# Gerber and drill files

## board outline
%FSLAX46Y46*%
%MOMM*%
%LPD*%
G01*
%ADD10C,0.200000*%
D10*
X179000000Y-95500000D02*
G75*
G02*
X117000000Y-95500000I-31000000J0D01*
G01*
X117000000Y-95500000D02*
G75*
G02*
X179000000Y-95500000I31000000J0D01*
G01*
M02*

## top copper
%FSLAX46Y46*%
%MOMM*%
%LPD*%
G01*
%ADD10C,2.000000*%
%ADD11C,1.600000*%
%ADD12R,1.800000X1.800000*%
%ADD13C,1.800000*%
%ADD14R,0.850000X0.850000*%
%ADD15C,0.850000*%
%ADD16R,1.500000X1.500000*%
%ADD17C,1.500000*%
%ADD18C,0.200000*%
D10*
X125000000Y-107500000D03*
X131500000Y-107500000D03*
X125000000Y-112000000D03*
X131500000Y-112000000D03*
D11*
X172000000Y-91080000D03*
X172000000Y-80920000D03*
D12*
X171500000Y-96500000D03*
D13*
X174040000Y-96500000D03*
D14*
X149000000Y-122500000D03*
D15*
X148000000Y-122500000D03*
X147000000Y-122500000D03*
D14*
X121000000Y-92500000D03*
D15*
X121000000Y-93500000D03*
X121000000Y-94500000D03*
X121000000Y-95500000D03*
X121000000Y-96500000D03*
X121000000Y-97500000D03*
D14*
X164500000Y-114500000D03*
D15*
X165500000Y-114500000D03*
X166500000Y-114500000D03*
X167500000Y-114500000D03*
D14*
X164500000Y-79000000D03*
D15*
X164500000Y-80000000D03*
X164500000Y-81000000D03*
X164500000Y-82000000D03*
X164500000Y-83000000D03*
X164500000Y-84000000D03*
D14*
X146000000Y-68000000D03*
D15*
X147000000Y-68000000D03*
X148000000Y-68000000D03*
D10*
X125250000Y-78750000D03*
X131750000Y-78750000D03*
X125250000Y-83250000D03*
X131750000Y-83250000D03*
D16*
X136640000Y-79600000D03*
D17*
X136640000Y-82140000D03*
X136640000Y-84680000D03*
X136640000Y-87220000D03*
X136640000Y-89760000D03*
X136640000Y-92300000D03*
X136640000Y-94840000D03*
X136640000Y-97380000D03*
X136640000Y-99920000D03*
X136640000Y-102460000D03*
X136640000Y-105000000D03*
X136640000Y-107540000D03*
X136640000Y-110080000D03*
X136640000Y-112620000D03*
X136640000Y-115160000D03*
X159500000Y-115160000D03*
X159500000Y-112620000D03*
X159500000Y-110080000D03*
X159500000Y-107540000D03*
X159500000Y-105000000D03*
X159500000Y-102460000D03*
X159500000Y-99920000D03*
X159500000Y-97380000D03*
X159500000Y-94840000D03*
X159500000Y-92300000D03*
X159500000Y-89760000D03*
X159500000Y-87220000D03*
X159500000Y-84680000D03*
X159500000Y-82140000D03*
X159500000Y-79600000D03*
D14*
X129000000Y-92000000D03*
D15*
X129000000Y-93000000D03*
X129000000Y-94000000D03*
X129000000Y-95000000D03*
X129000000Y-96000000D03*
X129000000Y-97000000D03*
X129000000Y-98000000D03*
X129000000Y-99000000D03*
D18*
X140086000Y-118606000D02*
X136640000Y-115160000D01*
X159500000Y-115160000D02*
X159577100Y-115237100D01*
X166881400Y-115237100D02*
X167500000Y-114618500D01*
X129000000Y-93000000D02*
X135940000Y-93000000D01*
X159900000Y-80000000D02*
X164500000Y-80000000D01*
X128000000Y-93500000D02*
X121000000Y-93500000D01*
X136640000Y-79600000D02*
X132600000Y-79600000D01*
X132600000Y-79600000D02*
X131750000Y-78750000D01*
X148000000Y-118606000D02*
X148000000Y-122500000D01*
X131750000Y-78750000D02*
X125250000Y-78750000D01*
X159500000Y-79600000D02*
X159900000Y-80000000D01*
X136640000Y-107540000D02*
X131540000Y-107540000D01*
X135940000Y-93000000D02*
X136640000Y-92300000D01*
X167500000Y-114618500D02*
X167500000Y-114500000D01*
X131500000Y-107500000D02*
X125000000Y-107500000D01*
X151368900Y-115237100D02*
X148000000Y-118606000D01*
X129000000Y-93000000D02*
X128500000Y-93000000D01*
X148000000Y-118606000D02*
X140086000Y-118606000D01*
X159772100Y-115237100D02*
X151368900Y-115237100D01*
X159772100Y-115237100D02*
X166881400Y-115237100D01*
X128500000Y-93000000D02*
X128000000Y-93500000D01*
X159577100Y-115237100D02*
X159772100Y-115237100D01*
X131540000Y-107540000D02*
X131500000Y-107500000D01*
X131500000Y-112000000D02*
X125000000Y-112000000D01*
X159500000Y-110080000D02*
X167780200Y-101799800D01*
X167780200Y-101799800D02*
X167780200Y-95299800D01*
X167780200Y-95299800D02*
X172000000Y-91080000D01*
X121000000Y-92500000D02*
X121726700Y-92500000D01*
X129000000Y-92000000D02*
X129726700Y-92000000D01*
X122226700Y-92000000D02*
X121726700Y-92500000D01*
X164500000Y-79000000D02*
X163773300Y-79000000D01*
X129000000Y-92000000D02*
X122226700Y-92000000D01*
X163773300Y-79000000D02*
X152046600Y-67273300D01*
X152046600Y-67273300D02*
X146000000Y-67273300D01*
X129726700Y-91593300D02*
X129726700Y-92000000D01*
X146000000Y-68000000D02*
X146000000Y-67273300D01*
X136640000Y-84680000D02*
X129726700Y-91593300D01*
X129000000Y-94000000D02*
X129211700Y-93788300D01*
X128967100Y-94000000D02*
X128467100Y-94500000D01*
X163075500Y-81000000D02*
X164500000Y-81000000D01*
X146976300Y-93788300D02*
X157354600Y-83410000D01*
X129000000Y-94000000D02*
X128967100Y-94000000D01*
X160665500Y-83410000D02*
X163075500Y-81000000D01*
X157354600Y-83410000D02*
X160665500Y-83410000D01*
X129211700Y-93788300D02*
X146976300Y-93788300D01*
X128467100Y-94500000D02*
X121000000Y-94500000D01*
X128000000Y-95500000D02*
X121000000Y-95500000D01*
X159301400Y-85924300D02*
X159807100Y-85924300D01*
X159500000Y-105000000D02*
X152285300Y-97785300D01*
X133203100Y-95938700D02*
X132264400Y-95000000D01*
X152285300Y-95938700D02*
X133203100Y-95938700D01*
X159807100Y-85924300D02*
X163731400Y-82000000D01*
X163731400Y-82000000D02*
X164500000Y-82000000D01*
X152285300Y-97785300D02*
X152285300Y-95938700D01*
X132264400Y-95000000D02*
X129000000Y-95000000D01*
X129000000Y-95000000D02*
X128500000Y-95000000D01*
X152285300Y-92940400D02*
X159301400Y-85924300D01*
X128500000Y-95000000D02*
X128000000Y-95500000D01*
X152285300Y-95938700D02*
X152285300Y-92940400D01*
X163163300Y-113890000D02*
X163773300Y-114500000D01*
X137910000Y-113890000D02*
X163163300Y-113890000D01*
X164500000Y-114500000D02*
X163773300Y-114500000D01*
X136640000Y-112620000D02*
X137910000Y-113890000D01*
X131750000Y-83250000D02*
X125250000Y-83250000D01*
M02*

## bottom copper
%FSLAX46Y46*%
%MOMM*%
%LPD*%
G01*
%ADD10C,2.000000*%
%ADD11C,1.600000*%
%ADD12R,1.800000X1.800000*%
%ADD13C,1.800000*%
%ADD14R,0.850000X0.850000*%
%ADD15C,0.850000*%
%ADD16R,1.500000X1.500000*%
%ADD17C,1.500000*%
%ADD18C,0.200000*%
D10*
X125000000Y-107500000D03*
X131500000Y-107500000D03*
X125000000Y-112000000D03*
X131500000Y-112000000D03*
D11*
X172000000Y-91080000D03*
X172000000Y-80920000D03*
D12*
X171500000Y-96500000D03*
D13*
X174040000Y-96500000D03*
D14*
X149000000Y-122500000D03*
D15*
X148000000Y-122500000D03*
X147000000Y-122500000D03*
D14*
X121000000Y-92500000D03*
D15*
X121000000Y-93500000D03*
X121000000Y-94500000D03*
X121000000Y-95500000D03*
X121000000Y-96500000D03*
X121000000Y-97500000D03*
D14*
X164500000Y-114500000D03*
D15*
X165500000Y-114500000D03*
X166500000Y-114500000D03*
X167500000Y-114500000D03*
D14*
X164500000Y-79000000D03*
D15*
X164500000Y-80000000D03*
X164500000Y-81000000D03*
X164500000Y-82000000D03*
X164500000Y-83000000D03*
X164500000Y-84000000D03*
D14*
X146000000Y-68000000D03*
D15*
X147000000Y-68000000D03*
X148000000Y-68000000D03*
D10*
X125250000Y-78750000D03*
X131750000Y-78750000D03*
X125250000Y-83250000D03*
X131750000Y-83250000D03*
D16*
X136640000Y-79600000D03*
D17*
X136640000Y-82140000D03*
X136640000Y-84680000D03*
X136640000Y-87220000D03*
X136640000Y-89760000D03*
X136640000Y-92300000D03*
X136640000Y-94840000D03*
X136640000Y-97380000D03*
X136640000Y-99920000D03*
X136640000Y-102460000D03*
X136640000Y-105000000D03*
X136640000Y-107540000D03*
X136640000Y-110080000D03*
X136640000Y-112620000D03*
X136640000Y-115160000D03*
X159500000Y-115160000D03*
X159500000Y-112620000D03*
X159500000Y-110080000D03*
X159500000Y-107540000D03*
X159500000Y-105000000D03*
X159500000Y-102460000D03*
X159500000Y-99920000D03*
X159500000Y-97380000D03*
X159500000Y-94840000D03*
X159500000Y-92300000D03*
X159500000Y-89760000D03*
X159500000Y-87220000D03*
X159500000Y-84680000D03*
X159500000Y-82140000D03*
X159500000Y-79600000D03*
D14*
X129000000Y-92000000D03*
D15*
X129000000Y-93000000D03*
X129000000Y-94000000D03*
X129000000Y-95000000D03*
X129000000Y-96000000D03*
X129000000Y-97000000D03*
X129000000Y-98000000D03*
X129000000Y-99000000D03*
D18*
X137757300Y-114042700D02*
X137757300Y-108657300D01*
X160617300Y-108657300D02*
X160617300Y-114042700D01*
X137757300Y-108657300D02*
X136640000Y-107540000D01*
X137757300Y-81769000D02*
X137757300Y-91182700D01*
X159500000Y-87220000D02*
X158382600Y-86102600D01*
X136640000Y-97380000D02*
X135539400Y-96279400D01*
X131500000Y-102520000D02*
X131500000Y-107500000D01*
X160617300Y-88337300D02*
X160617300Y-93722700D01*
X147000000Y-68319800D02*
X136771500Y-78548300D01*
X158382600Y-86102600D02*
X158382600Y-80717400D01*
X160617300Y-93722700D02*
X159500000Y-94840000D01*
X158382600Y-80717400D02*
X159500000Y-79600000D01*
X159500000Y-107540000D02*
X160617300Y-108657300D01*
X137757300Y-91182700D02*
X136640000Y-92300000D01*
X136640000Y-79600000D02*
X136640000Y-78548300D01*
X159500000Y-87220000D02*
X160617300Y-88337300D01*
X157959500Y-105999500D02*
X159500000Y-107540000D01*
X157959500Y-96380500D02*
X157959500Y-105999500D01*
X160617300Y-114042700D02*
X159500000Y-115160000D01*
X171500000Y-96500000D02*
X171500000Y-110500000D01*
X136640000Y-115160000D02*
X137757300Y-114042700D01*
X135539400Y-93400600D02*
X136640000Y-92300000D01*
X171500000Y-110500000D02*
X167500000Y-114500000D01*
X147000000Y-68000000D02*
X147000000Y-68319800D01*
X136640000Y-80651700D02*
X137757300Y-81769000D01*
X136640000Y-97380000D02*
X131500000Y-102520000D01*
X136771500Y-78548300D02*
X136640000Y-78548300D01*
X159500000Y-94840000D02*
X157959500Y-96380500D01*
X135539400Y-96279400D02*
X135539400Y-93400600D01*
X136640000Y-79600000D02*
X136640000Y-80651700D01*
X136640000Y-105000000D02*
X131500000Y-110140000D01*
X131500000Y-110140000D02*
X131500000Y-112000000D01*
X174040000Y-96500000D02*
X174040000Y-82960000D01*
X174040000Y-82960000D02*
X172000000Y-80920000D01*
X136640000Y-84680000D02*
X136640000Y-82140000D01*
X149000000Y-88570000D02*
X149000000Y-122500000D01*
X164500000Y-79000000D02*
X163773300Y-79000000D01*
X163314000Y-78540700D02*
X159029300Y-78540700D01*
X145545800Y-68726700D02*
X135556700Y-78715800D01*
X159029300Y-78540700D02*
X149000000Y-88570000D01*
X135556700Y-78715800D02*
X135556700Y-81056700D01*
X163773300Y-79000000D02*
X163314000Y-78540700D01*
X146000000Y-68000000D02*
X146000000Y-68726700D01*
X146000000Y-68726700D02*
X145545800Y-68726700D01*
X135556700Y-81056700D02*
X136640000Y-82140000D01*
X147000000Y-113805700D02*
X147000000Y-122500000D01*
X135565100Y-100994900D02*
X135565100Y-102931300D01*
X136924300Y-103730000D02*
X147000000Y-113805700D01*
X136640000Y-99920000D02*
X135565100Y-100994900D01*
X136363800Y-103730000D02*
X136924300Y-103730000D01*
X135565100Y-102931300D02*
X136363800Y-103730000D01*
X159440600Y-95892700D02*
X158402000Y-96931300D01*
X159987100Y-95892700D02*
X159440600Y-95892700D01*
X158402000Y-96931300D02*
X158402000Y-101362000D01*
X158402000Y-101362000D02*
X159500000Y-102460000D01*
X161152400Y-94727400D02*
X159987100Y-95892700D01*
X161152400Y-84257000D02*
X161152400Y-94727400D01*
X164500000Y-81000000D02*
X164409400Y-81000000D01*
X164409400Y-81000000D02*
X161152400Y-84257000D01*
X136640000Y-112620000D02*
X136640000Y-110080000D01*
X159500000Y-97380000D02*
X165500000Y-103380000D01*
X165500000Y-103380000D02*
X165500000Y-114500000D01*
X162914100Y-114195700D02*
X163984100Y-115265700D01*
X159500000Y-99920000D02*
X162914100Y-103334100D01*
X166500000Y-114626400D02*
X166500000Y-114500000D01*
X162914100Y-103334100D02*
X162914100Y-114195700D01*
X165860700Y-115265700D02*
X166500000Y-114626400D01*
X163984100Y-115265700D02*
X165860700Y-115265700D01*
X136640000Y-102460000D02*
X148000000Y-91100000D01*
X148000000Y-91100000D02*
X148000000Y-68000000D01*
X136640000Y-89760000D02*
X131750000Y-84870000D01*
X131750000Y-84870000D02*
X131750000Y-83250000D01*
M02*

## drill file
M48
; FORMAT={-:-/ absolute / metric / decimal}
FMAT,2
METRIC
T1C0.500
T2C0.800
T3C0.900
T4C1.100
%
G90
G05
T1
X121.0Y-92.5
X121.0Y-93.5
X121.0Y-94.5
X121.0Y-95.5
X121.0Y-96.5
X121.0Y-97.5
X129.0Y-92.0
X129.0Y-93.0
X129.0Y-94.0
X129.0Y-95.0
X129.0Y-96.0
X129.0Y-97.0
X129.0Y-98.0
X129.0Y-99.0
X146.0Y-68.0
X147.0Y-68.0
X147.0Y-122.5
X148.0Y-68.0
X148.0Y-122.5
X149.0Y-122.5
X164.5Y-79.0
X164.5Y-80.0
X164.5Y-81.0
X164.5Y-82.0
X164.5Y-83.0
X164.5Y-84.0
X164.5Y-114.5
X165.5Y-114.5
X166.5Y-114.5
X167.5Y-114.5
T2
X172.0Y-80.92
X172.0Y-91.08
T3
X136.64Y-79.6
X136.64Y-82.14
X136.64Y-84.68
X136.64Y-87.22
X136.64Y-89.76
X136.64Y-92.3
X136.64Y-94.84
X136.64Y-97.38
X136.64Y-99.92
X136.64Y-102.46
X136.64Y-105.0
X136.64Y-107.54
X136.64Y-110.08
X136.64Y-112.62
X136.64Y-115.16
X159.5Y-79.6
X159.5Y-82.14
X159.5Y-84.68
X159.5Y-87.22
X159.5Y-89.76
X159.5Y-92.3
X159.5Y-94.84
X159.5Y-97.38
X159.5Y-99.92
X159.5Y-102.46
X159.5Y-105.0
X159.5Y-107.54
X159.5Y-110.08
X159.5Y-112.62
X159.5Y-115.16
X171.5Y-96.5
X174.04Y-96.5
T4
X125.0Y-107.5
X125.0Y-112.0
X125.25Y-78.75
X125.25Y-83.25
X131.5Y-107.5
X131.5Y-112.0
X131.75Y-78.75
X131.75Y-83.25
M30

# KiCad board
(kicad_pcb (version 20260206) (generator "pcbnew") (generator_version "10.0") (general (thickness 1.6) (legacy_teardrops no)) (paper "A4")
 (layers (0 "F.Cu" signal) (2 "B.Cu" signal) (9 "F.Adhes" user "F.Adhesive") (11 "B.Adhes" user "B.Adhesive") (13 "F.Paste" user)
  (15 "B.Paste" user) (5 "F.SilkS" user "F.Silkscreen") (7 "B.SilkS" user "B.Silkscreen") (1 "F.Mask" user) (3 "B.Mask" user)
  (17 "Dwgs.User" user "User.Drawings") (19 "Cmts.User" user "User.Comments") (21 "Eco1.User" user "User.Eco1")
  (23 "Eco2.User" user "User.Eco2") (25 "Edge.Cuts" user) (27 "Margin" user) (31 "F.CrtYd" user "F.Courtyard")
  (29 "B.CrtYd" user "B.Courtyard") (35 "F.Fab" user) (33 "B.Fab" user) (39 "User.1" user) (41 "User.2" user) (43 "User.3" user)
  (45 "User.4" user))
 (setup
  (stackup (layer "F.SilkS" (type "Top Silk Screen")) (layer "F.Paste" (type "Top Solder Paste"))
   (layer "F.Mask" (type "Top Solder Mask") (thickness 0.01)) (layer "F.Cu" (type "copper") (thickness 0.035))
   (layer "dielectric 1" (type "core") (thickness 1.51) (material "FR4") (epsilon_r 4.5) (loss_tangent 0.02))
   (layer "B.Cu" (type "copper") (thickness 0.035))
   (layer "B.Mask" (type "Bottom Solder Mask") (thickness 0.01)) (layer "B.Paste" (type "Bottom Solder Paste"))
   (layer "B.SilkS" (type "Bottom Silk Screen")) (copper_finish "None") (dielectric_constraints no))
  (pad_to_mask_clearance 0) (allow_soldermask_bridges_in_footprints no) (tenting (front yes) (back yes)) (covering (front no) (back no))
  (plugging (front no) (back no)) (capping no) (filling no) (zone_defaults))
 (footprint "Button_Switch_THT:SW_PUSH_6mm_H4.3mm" (layer "F.Cu") (at 125 107.5)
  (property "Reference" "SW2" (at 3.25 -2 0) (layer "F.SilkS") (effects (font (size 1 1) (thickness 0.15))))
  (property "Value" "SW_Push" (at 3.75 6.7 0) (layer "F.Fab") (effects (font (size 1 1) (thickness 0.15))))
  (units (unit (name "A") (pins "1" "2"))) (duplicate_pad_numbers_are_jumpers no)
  (pad "1" thru_hole circle (at 0 0 90) (size 2 2) (drill 1.1) (layers "*.Cu" "*.Mask") (remove_unused_layers no) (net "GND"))
  (pad "1" thru_hole circle (at 6.5 0 90) (size 2 2) (drill 1.1) (layers "*.Cu" "*.Mask") (remove_unused_layers no) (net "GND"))
  (pad "2" thru_hole circle (at 0 4.5 90) (size 2 2) (drill 1.1) (layers "*.Cu" "*.Mask") (remove_unused_layers no) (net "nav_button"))
  (pad "2" thru_hole circle (at 6.5 4.5 90) (size 2 2) (drill 1.1) (layers "*.Cu" "*.Mask") (remove_unused_layers no) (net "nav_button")))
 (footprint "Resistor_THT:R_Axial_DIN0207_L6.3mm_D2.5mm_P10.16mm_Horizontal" (layer "F.Cu") (at 172 91.08 90)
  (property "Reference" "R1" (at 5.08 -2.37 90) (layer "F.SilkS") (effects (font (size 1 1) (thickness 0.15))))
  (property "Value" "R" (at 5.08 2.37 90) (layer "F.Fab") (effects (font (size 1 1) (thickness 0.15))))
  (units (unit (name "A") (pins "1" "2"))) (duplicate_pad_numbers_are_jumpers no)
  (pad "1" thru_hole circle (at 0 0 90) (size 1.6 1.6) (drill 0.8) (layers "*.Cu" "*.Mask") (remove_unused_layers no) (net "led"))
  (pad "2" thru_hole circle (at 10.16 0 90) (size 1.6 1.6) (drill 0.8) (layers "*.Cu" "*.Mask") (remove_unused_layers no) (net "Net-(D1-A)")))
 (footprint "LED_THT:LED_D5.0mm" (layer "F.Cu") (at 171.5 96.5)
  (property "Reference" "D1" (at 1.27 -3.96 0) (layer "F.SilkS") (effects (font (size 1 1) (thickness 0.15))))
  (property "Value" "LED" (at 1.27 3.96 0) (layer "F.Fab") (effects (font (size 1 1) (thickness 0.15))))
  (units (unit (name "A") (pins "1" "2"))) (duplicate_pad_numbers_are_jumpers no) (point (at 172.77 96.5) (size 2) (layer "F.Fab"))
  (pad "1" thru_hole rect (at 0 0) (size 1.8 1.8) (drill 0.9) (layers "*.Cu" "*.Mask") (remove_unused_layers no) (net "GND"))
  (pad "2" thru_hole circle (at 2.54 0) (size 1.8 1.8) (drill 0.9) (layers "*.Cu" "*.Mask") (remove_unused_layers no) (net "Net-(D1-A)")))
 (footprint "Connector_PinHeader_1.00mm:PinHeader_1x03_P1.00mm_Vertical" (layer "F.Cu") (at 149 122.5 -90)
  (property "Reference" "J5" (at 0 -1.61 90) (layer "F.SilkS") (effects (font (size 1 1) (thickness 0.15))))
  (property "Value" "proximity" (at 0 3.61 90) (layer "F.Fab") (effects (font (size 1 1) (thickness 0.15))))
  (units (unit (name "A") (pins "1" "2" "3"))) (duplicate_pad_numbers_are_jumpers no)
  (pad "1" thru_hole rect (at 0 0 270) (size 0.85 0.85) (drill 0.5) (layers "*.Cu" "*.Mask") (remove_unused_layers no) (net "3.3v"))
  (pad "2" thru_hole circle (at 0 1 270) (size 0.85 0.85) (drill 0.5) (layers "*.Cu" "*.Mask") (remove_unused_layers no) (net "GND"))
  (pad "3" thru_hole circle (at 0 2 270) (size 0.85 0.85) (drill 0.5) (layers "*.Cu" "*.Mask") (remove_unused_layers no) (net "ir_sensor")))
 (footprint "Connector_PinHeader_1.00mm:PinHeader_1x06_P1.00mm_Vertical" (layer "F.Cu") (at 121 92.5)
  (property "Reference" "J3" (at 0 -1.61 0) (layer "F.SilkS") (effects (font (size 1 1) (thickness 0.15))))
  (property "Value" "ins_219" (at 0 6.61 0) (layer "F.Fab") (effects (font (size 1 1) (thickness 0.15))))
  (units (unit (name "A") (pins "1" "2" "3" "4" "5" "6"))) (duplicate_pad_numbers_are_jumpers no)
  (pad "1" thru_hole rect (at 0 0) (size 0.85 0.85) (drill 0.5) (layers "*.Cu" "*.Mask") (remove_unused_layers no) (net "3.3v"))
  (pad "2" thru_hole circle (at 0 1) (size 0.85 0.85) (drill 0.5) (layers "*.Cu" "*.Mask") (remove_unused_layers no) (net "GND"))
  (pad "3" thru_hole circle (at 0 2) (size 0.85 0.85) (drill 0.5) (layers "*.Cu" "*.Mask") (remove_unused_layers no) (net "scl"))
  (pad "4" thru_hole circle (at 0 3) (size 0.85 0.85) (drill 0.5) (layers "*.Cu" "*.Mask") (remove_unused_layers no) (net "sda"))
  (pad "5" thru_hole circle (at 0 4) (size 0.85 0.85) (drill 0.5) (layers "*.Cu" "*.Mask") (remove_unused_layers no)
   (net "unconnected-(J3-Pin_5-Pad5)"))
  (pad "6" thru_hole circle (at 0 5) (size 0.85 0.85) (drill 0.5) (layers "*.Cu" "*.Mask") (remove_unused_layers no)
   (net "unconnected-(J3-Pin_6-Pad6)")))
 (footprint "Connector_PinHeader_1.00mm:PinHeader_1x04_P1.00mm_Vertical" (layer "F.Cu") (at 164.5 114.5 90)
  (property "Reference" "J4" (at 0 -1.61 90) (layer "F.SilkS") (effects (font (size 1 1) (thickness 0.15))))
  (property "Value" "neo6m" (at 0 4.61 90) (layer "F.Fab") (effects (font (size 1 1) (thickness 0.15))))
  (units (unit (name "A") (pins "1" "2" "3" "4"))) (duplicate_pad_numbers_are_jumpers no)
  (pad "1" thru_hole rect (at 0 0 90) (size 0.85 0.85) (drill 0.5) (layers "*.Cu" "*.Mask") (remove_unused_layers no) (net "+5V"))
  (pad "2" thru_hole circle (at 0 1 90) (size 0.85 0.85) (drill 0.5) (layers "*.Cu" "*.Mask") (remove_unused_layers no) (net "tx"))
  (pad "3" thru_hole circle (at 0 2 90) (size 0.85 0.85) (drill 0.5) (layers "*.Cu" "*.Mask") (remove_unused_layers no) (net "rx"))
  (pad "4" thru_hole circle (at 0 3 90) (size 0.85 0.85) (drill 0.5) (layers "*.Cu" "*.Mask") (remove_unused_layers no) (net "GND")))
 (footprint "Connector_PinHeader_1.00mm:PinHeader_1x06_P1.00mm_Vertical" (layer "F.Cu") (at 164.5 79)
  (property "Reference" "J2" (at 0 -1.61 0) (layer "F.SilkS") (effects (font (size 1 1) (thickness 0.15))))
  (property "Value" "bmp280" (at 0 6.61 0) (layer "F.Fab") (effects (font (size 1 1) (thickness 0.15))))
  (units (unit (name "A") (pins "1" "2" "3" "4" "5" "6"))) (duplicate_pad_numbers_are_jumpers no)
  (pad "1" thru_hole rect (at 0 0) (size 0.85 0.85) (drill 0.5) (layers "*.Cu" "*.Mask") (remove_unused_layers no) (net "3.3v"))
  (pad "2" thru_hole circle (at 0 1) (size 0.85 0.85) (drill 0.5) (layers "*.Cu" "*.Mask") (remove_unused_layers no) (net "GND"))
  (pad "3" thru_hole circle (at 0 2) (size 0.85 0.85) (drill 0.5) (layers "*.Cu" "*.Mask") (remove_unused_layers no) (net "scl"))
  (pad "4" thru_hole circle (at 0 3) (size 0.85 0.85) (drill 0.5) (layers "*.Cu" "*.Mask") (remove_unused_layers no) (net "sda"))
  (pad "5" thru_hole circle (at 0 4) (size 0.85 0.85) (drill 0.5) (layers "*.Cu" "*.Mask") (remove_unused_layers no)
   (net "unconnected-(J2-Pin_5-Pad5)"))
  (pad "6" thru_hole circle (at 0 5) (size 0.85 0.85) (drill 0.5) (layers "*.Cu" "*.Mask") (remove_unused_layers no)
   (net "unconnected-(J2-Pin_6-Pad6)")))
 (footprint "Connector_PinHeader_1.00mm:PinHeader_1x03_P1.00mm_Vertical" (layer "F.Cu") (at 146 68 90)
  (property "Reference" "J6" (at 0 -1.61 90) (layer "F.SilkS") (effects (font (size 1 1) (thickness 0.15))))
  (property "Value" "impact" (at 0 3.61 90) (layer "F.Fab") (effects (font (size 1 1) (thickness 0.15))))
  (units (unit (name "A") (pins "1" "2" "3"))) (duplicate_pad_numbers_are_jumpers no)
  (pad "1" thru_hole rect (at 0 0 90) (size 0.85 0.85) (drill 0.5) (layers "*.Cu" "*.Mask") (remove_unused_layers no) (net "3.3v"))
  (pad "2" thru_hole circle (at 0 1 90) (size 0.85 0.85) (drill 0.5) (layers "*.Cu" "*.Mask") (remove_unused_layers no) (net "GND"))
  (pad "3" thru_hole circle (at 0 2 90) (size 0.85 0.85) (drill 0.5) (layers "*.Cu" "*.Mask") (remove_unused_layers no) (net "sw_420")))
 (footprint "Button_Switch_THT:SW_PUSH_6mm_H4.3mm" (layer "F.Cu") (at 125.25 78.75)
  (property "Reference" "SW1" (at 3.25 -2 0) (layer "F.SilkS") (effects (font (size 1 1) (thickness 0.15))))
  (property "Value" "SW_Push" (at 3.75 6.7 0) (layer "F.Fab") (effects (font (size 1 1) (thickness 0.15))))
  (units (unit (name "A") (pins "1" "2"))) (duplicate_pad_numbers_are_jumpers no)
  (pad "1" thru_hole circle (at 0 0 90) (size 2 2) (drill 1.1) (layers "*.Cu" "*.Mask") (remove_unused_layers no) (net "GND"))
  (pad "1" thru_hole circle (at 6.5 0 90) (size 2 2) (drill 1.1) (layers "*.Cu" "*.Mask") (remove_unused_layers no) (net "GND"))
  (pad "2" thru_hole circle (at 0 4.5 90) (size 2 2) (drill 1.1) (layers "*.Cu" "*.Mask") (remove_unused_layers no) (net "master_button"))
  (pad "2" thru_hole circle (at 6.5 4.5 90) (size 2 2) (drill 1.1) (layers "*.Cu" "*.Mask") (remove_unused_layers no) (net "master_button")))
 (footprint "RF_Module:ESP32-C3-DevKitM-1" (layer "F.Cu") (at 136.64 79.6)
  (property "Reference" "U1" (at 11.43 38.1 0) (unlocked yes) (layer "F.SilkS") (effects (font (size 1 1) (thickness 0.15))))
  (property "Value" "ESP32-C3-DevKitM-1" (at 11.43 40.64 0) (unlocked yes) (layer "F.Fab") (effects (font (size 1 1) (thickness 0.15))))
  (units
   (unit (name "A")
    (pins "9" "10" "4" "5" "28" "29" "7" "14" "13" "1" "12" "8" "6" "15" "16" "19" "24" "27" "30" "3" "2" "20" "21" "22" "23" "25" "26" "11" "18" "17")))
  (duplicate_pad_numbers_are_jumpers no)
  (pad "1" thru_hole rect (at 0 0) (size 1.5 1.5) (drill 0.9) (layers "*.Cu" "*.Mask") (remove_unused_layers yes) (keep_end_layers yes)
   (zone_layer_connections) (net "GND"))
  (pad "2" thru_hole circle (at 0 2.54) (size 1.5 1.5) (drill 0.9) (layers "*.Cu" "*.Mask") (remove_unused_layers yes) (keep_end_layers yes)
   (zone_layer_connections) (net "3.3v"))
  (pad "3" thru_hole circle (at 0 5.08) (size 1.5 1.5) (drill 0.9) (layers "*.Cu" "*.Mask") (remove_unused_layers yes) (keep_end_layers yes)
   (zone_layer_connections) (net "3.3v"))
  (pad "4" thru_hole circle (at 0 7.62) (size 1.5 1.5) (drill 0.9) (layers "*.Cu" "*.Mask") (remove_unused_layers yes) (keep_end_layers yes)
   (zone_layer_connections) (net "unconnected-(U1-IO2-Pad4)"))
  (pad "5" thru_hole circle (at 0 10.16) (size 1.5 1.5) (drill 0.9) (layers "*.Cu" "*.Mask") (remove_unused_layers yes)
   (keep_end_layers yes) (zone_layer_connections) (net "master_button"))
  (pad "6" thru_hole circle (at 0 12.7) (size 1.5 1.5) (drill 0.9) (layers "*.Cu" "*.Mask") (remove_unused_layers yes) (keep_end_layers yes)
   (zone_layer_connections) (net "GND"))
  (pad "7" thru_hole circle (at 0 15.24) (size 1.5 1.5) (drill 0.9) (layers "*.Cu" "*.Mask") (remove_unused_layers yes)
   (keep_end_layers yes) (zone_layer_connections) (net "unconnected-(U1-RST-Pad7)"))
  (pad "8" thru_hole circle (at 0 17.78) (size 1.5 1.5) (drill 0.9) (layers "*.Cu" "*.Mask") (remove_unused_layers yes)
   (keep_end_layers yes) (zone_layer_connections) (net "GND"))
  (pad "9" thru_hole circle (at 0 20.32) (size 1.5 1.5) (drill 0.9) (layers "*.Cu" "*.Mask") (remove_unused_layers yes)
   (keep_end_layers yes) (zone_layer_connections) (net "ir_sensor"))
  (pad "10" thru_hole circle (at 0 22.86) (size 1.5 1.5) (drill 0.9) (layers "*.Cu" "*.Mask") (remove_unused_layers yes)
   (keep_end_layers yes) (zone_layer_connections) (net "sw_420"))
  (pad "11" thru_hole circle (at 0 25.4) (size 1.5 1.5) (drill 0.9) (layers "*.Cu" "*.Mask") (remove_unused_layers yes)
   (keep_end_layers yes) (zone_layer_connections) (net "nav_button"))
  (pad "12" thru_hole circle (at 0 27.94) (size 1.5 1.5) (drill 0.9) (layers "*.Cu" "*.Mask") (remove_unused_layers yes)
   (keep_end_layers yes) (zone_layer_connections) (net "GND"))
  (pad "13" thru_hole circle (at 0 30.48) (size 1.5 1.5) (drill 0.9) (layers "*.Cu" "*.Mask") (remove_unused_layers yes)
   (keep_end_layers yes) (zone_layer_connections) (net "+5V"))
  (pad "14" thru_hole circle (at 0 33.02) (size 1.5 1.5) (drill 0.9) (layers "*.Cu" "*.Mask") (remove_unused_layers yes)
   (keep_end_layers yes) (zone_layer_connections) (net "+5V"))
  (pad "15" thru_hole circle (at 0 35.56) (size 1.5 1.5) (drill 0.9) (layers "*.Cu" "*.Mask") (remove_unused_layers yes)
   (keep_end_layers yes) (zone_layer_connections) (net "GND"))
  (pad "16" thru_hole circle (at 22.86 35.56) (size 1.5 1.5) (drill 0.9) (layers "*.Cu" "*.Mask") (remove_unused_layers yes)
   (keep_end_layers yes) (zone_layer_connections) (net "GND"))
  (pad "17" thru_hole circle (at 22.86 33.02) (size 1.5 1.5) (drill 0.9) (layers "*.Cu" "*.Mask") (remove_unused_layers yes)
   (keep_end_layers yes) (zone_layer_connections) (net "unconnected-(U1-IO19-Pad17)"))
  (pad "18" thru_hole circle (at 22.86 30.48) (size 1.5 1.5) (drill 0.9) (layers "*.Cu" "*.Mask") (remove_unused_layers yes)
   (keep_end_layers yes) (zone_layer_connections) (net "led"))
  (pad "19" thru_hole circle (at 22.86 27.94) (size 1.5 1.5) (drill 0.9) (layers "*.Cu" "*.Mask") (remove_unused_layers yes)
   (keep_end_layers yes) (zone_layer_connections) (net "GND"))
  (pad "20" thru_hole circle (at 22.86 25.4) (size 1.5 1.5) (drill 0.9) (layers "*.Cu" "*.Mask") (remove_unused_layers yes)
   (keep_end_layers yes) (zone_layer_connections) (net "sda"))
  (pad "21" thru_hole circle (at 22.86 22.86) (size 1.5 1.5) (drill 0.9) (layers "*.Cu" "*.Mask") (remove_unused_layers yes)
   (keep_end_layers yes) (zone_layer_connections) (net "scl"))
  (pad "22" thru_hole circle (at 22.86 20.32) (size 1.5 1.5) (drill 0.9) (layers "*.Cu" "*.Mask") (remove_unused_layers yes)
   (keep_end_layers yes) (zone_layer_connections) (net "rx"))
  (pad "23" thru_hole circle (at 22.86 17.78) (size 1.5 1.5) (drill 0.9) (layers "*.Cu" "*.Mask") (remove_unused_layers yes)
   (keep_end_layers yes) (zone_layer_connections) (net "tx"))
  (pad "24" thru_hole circle (at 22.86 15.24) (size 1.5 1.5) (drill 0.9) (layers "*.Cu" "*.Mask") (remove_unused_layers yes)
   (keep_end_layers yes) (zone_layer_connections) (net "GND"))
  (pad "25" thru_hole circle (at 22.86 12.7) (size 1.5 1.5) (drill 0.9) (layers "*.Cu" "*.Mask") (remove_unused_layers yes)
   (keep_end_layers yes) (zone_layer_connections) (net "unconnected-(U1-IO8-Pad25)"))
  (pad "26" thru_hole circle (at 22.86 10.16) (size 1.5 1.5) (drill 0.9) (layers "*.Cu" "*.Mask") (remove_unused_layers yes)
   (keep_end_layers yes) (zone_layer_connections) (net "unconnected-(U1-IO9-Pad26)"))
  (pad "27" thru_hole circle (at 22.86 7.62) (size 1.5 1.5) (drill 0.9) (layers "*.Cu" "*.Mask") (remove_unused_layers yes)
   (keep_end_layers yes) (zone_layer_connections) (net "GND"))
  (pad "28" thru_hole circle (at 22.86 5.08) (size 1.5 1.5) (drill 0.9) (layers "*.Cu" "*.Mask") (remove_unused_layers yes)
   (keep_end_layers yes) (zone_layer_connections) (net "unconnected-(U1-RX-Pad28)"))
  (pad "29" thru_hole circle (at 22.86 2.54) (size 1.5 1.5) (drill 0.9) (layers "*.Cu" "*.Mask") (remove_unused_layers yes)
   (keep_end_layers yes) (zone_layer_connections) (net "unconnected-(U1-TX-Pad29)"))
  (pad "30" thru_hole circle (at 22.86 0) (size 1.5 1.5) (drill 0.9) (layers "*.Cu" "*.Mask") (remove_unused_layers yes)
   (keep_end_layers yes) (zone_layer_connections) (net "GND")))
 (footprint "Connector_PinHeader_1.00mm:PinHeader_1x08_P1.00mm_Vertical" (layer "F.Cu") (at 129 92)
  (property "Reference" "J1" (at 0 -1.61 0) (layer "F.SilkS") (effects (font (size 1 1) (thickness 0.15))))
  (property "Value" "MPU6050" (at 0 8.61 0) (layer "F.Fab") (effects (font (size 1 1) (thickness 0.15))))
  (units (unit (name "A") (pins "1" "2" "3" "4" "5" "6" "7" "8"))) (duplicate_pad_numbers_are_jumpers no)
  (pad "1" thru_hole rect (at 0 0) (size 0.85 0.85) (drill 0.5) (layers "*.Cu" "*.Mask") (remove_unused_layers no) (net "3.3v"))
  (pad "2" thru_hole circle (at 0 1) (size 0.85 0.85) (drill 0.5) (layers "*.Cu" "*.Mask") (remove_unused_layers no) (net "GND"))
  (pad "3" thru_hole circle (at 0 2) (size 0.85 0.85) (drill 0.5) (layers "*.Cu" "*.Mask") (remove_unused_layers no) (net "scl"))
  (pad "4" thru_hole circle (at 0 3) (size 0.85 0.85) (drill 0.5) (layers "*.Cu" "*.Mask") (remove_unused_layers no) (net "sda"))
  (pad "5" thru_hole circle (at 0 4) (size 0.85 0.85) (drill 0.5) (layers "*.Cu" "*.Mask") (remove_unused_layers no)
   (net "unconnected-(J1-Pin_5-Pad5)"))
  (pad "6" thru_hole circle (at 0 5) (size 0.85 0.85) (drill 0.5) (layers "*.Cu" "*.Mask") (remove_unused_layers no)
   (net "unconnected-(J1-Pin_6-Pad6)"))
  (pad "7" thru_hole circle (at 0 6) (size 0.85 0.85) (drill 0.5) (layers "*.Cu" "*.Mask") (remove_unused_layers no)
   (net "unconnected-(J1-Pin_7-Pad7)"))
  (pad "8" thru_hole circle (at 0 7) (size 0.85 0.85) (drill 0.5) (layers "*.Cu" "*.Mask") (remove_unused_layers no)
   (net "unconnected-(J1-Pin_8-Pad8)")))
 (gr_circle (center 148 95.5) (end 179 95.5) (stroke (width 0.2) (type default)) (fill no) (layer "Edge.Cuts"))
 (segment (start 140.086 118.606) (end 136.64 115.16) (width 0.2) (layer "F.Cu") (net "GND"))
 (segment (start 159.5 115.16) (end 159.5771 115.2371) (width 0.2) (layer "F.Cu") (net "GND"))
 (segment (start 166.8814 115.2371) (end 167.5 114.6185) (width 0.2) (layer "F.Cu") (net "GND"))
 (segment (start 129 93) (end 135.94 93) (width 0.2) (layer "F.Cu") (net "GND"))
 (segment (start 159.9 80) (end 164.5 80) (width 0.2) (layer "F.Cu") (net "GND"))
 (segment (start 128 93.5) (end 121 93.5) (width 0.2) (layer "F.Cu") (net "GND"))
 (segment (start 136.64 79.6) (end 132.6 79.6) (width 0.2) (layer "F.Cu") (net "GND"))
 (segment (start 132.6 79.6) (end 131.75 78.75) (width 0.2) (layer "F.Cu") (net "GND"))
 (segment (start 148 118.606) (end 148 122.5) (width 0.2) (layer "F.Cu") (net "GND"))
 (segment (start 131.75 78.75) (end 125.25 78.75) (width 0.2) (layer "F.Cu") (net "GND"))
 (segment (start 159.5 79.6) (end 159.9 80) (width 0.2) (layer "F.Cu") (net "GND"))
 (segment (start 136.64 107.54) (end 131.54 107.54) (width 0.2) (layer "F.Cu") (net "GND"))
 (segment (start 135.94 93) (end 136.64 92.3) (width 0.2) (layer "F.Cu") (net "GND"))
 (segment (start 167.5 114.6185) (end 167.5 114.5) (width 0.2) (layer "F.Cu") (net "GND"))
 (segment (start 131.5 107.5) (end 125 107.5) (width 0.2) (layer "F.Cu") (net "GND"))
 (segment (start 151.3689 115.2371) (end 148 118.606) (width 0.2) (layer "F.Cu") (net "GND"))
 (segment (start 129 93) (end 128.5 93) (width 0.2) (layer "F.Cu") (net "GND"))
 (segment (start 148 118.606) (end 140.086 118.606) (width 0.2) (layer "F.Cu") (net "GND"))
 (segment (start 159.7721 115.2371) (end 151.3689 115.2371) (width 0.2) (layer "F.Cu") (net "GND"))
 (segment (start 159.7721 115.2371) (end 166.8814 115.2371) (width 0.2) (layer "F.Cu") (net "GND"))
 (segment (start 128.5 93) (end 128 93.5) (width 0.2) (layer "F.Cu") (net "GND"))
 (segment (start 159.5771 115.2371) (end 159.7721 115.2371) (width 0.2) (layer "F.Cu") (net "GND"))
 (segment (start 131.54 107.54) (end 131.5 107.5) (width 0.2) (layer "F.Cu") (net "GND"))
 (segment (start 137.7573 114.0427) (end 137.7573 108.6573) (width 0.2) (layer "B.Cu") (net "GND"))
 (segment (start 160.6173 108.6573) (end 160.6173 114.0427) (width 0.2) (layer "B.Cu") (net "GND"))
 (segment (start 137.7573 108.6573) (end 136.64 107.54) (width 0.2) (layer "B.Cu") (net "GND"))
 (segment (start 137.7573 81.769) (end 137.7573 91.1827) (width 0.2) (layer "B.Cu") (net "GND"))
 (segment (start 159.5 87.22) (end 158.3826 86.1026) (width 0.2) (layer "B.Cu") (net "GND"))
 (segment (start 136.64 97.38) (end 135.5394 96.2794) (width 0.2) (layer "B.Cu") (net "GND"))
 (segment (start 131.5 102.52) (end 131.5 107.5) (width 0.2) (layer "B.Cu") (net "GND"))
 (segment (start 160.6173 88.3373) (end 160.6173 93.7227) (width 0.2) (layer "B.Cu") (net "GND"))
 (segment (start 147 68.3198) (end 136.7715 78.5483) (width 0.2) (layer "B.Cu") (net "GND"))
 (segment (start 158.3826 86.1026) (end 158.3826 80.7174) (width 0.2) (layer "B.Cu") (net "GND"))
 (segment (start 160.6173 93.7227) (end 159.5 94.84) (width 0.2) (layer "B.Cu") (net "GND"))
 (segment (start 158.3826 80.7174) (end 159.5 79.6) (width 0.2) (layer "B.Cu") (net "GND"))
 (segment (start 159.5 107.54) (end 160.6173 108.6573) (width 0.2) (layer "B.Cu") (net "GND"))
 (segment (start 137.7573 91.1827) (end 136.64 92.3) (width 0.2) (layer "B.Cu") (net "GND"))
 (segment (start 136.64 79.6) (end 136.64 78.5483) (width 0.2) (layer "B.Cu") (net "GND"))
 (segment (start 159.5 87.22) (end 160.6173 88.3373) (width 0.2) (layer "B.Cu") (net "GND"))
 (segment (start 157.9595 105.9995) (end 159.5 107.54) (width 0.2) (layer "B.Cu") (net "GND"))
 (segment (start 157.9595 96.3805) (end 157.9595 105.9995) (width 0.2) (layer "B.Cu") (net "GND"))
 (segment (start 160.6173 114.0427) (end 159.5 115.16) (width 0.2) (layer "B.Cu") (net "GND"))
 (segment (start 171.5 96.5) (end 171.5 110.5) (width 0.2) (layer "B.Cu") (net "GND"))
 (segment (start 136.64 115.16) (end 137.7573 114.0427) (width 0.2) (layer "B.Cu") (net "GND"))
 (segment (start 135.5394 93.4006) (end 136.64 92.3) (width 0.2) (layer "B.Cu") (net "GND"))
 (segment (start 171.5 110.5) (end 167.5 114.5) (width 0.2) (layer "B.Cu") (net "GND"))
 (segment (start 147 68) (end 147 68.3198) (width 0.2) (layer "B.Cu") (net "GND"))
 (segment (start 136.64 80.6517) (end 137.7573 81.769) (width 0.2) (layer "B.Cu") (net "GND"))
 (segment (start 136.64 97.38) (end 131.5 102.52) (width 0.2) (layer "B.Cu") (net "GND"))
 (segment (start 136.7715 78.5483) (end 136.64 78.5483) (width 0.2) (layer "B.Cu") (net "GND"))
 (segment (start 159.5 94.84) (end 157.9595 96.3805) (width 0.2) (layer "B.Cu") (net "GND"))
 (segment (start 135.5394 96.2794) (end 135.5394 93.4006) (width 0.2) (layer "B.Cu") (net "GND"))
 (segment (start 136.64 79.6) (end 136.64 80.6517) (width 0.2) (layer "B.Cu") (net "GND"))
 (segment (start 131.5 112) (end 125 112) (width 0.2) (layer "F.Cu") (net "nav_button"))
 (segment (start 136.64 105) (end 131.5 110.14) (width 0.2) (layer "B.Cu") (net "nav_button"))
 (segment (start 131.5 110.14) (end 131.5 112) (width 0.2) (layer "B.Cu") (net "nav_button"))
 (segment (start 159.5 110.08) (end 167.7802 101.7998) (width 0.2) (layer "F.Cu") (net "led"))
 (segment (start 167.7802 101.7998) (end 167.7802 95.2998) (width 0.2) (layer "F.Cu") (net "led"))
 (segment (start 167.7802 95.2998) (end 172 91.08) (width 0.2) (layer "F.Cu") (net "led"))
 (segment (start 174.04 96.5) (end 174.04 82.96) (width 0.2) (layer "B.Cu") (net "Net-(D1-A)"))
 (segment (start 174.04 82.96) (end 172 80.92) (width 0.2) (layer "B.Cu") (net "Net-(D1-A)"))
 (segment (start 121 92.5) (end 121.7267 92.5) (width 0.2) (layer "F.Cu") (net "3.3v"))
 (segment (start 129 92) (end 129.7267 92) (width 0.2) (layer "F.Cu") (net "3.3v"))
 (segment (start 122.2267 92) (end 121.7267 92.5) (width 0.2) (layer "F.Cu") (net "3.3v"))
 (segment (start 164.5 79) (end 163.7733 79) (width 0.2) (layer "F.Cu") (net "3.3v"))
 (segment (start 129 92) (end 122.2267 92) (width 0.2) (layer "F.Cu") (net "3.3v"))
 (segment (start 163.7733 79) (end 152.0466 67.2733) (width 0.2) (layer "F.Cu") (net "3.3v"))
 (segment (start 152.0466 67.2733) (end 146 67.2733) (width 0.2) (layer "F.Cu") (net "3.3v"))
 (segment (start 129.7267 91.5933) (end 129.7267 92) (width 0.2) (layer "F.Cu") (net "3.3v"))
 (segment (start 146 68) (end 146 67.2733) (width 0.2) (layer "F.Cu") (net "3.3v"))
 (segment (start 136.64 84.68) (end 129.7267 91.5933) (width 0.2) (layer "F.Cu") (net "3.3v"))
 (segment (start 136.64 84.68) (end 136.64 82.14) (width 0.2) (layer "B.Cu") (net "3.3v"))
 (segment (start 149 88.57) (end 149 122.5) (width 0.2) (layer "B.Cu") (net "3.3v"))
 (segment (start 164.5 79) (end 163.7733 79) (width 0.2) (layer "B.Cu") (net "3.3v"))
 (segment (start 163.314 78.5407) (end 159.0293 78.5407) (width 0.2) (layer "B.Cu") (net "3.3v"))
 (segment (start 145.5458 68.7267) (end 135.5567 78.7158) (width 0.2) (layer "B.Cu") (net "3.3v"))
 (segment (start 159.0293 78.5407) (end 149 88.57) (width 0.2) (layer "B.Cu") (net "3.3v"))
 (segment (start 135.5567 78.7158) (end 135.5567 81.0567) (width 0.2) (layer "B.Cu") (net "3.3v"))
 (segment (start 163.7733 79) (end 163.314 78.5407) (width 0.2) (layer "B.Cu") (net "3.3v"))
 (segment (start 146 68) (end 146 68.7267) (width 0.2) (layer "B.Cu") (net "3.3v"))
 (segment (start 146 68.7267) (end 145.5458 68.7267) (width 0.2) (layer "B.Cu") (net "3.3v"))
 (segment (start 135.5567 81.0567) (end 136.64 82.14) (width 0.2) (layer "B.Cu") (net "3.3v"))
 (segment (start 147 113.8057) (end 147 122.5) (width 0.2) (layer "B.Cu") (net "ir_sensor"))
 (segment (start 135.5651 100.9949) (end 135.5651 102.9313) (width 0.2) (layer "B.Cu") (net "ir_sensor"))
 (segment (start 136.9243 103.73) (end 147 113.8057) (width 0.2) (layer "B.Cu") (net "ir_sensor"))
 (segment (start 136.64 99.92) (end 135.5651 100.9949) (width 0.2) (layer "B.Cu") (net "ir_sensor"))
 (segment (start 136.3638 103.73) (end 136.9243 103.73) (width 0.2) (layer "B.Cu") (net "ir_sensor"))
 (segment (start 135.5651 102.9313) (end 136.3638 103.73) (width 0.2) (layer "B.Cu") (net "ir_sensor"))
 (segment (start 129 94) (end 129.2117 93.7883) (width 0.2) (layer "F.Cu") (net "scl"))
 (segment (start 128.9671 94) (end 128.4671 94.5) (width 0.2) (layer "F.Cu") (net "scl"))
 (segment (start 163.0755 81) (end 164.5 81) (width 0.2) (layer "F.Cu") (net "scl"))
 (segment (start 146.9763 93.7883) (end 157.3546 83.41) (width 0.2) (layer "F.Cu") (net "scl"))
 (segment (start 129 94) (end 128.9671 94) (width 0.2) (layer "F.Cu") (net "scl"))
 (segment (start 160.6655 83.41) (end 163.0755 81) (width 0.2) (layer "F.Cu") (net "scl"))
 (segment (start 157.3546 83.41) (end 160.6655 83.41) (width 0.2) (layer "F.Cu") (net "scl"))
 (segment (start 129.2117 93.7883) (end 146.9763 93.7883) (width 0.2) (layer "F.Cu") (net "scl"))
 (segment (start 128.4671 94.5) (end 121 94.5) (width 0.2) (layer "F.Cu") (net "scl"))
 (segment (start 159.4406 95.8927) (end 158.402 96.9313) (width 0.2) (layer "B.Cu") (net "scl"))
 (segment (start 159.9871 95.8927) (end 159.4406 95.8927) (width 0.2) (layer "B.Cu") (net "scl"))
 (segment (start 158.402 96.9313) (end 158.402 101.362) (width 0.2) (layer "B.Cu") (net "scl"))
 (segment (start 158.402 101.362) (end 159.5 102.46) (width 0.2) (layer "B.Cu") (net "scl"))
 (segment (start 161.1524 94.7274) (end 159.9871 95.8927) (width 0.2) (layer "B.Cu") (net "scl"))
 (segment (start 161.1524 84.257) (end 161.1524 94.7274) (width 0.2) (layer "B.Cu") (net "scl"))
 (segment (start 164.5 81) (end 164.4094 81) (width 0.2) (layer "B.Cu") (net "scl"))
 (segment (start 164.4094 81) (end 161.1524 84.257) (width 0.2) (layer "B.Cu") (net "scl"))
 (segment (start 128 95.5) (end 121 95.5) (width 0.2) (layer "F.Cu") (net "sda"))
 (segment (start 159.3014 85.9243) (end 159.8071 85.9243) (width 0.2) (layer "F.Cu") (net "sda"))
 (segment (start 159.5 105) (end 152.2853 97.7853) (width 0.2) (layer "F.Cu") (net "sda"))
 (segment (start 133.2031 95.9387) (end 132.2644 95) (width 0.2) (layer "F.Cu") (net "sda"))
 (segment (start 152.2853 95.9387) (end 133.2031 95.9387) (width 0.2) (layer "F.Cu") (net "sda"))
 (segment (start 159.8071 85.9243) (end 163.7314 82) (width 0.2) (layer "F.Cu") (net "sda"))
 (segment (start 163.7314 82) (end 164.5 82) (width 0.2) (layer "F.Cu") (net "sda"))
 (segment (start 152.2853 97.7853) (end 152.2853 95.9387) (width 0.2) (layer "F.Cu") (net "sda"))
 (segment (start 132.2644 95) (end 129 95) (width 0.2) (layer "F.Cu") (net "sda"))
 (segment (start 129 95) (end 128.5 95) (width 0.2) (layer "F.Cu") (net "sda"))
 (segment (start 152.2853 92.9404) (end 159.3014 85.9243) (width 0.2) (layer "F.Cu") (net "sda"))
 (segment (start 128.5 95) (end 128 95.5) (width 0.2) (layer "F.Cu") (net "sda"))
 (segment (start 152.2853 95.9387) (end 152.2853 92.9404) (width 0.2) (layer "F.Cu") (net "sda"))
 (segment (start 163.1633 113.89) (end 163.7733 114.5) (width 0.2) (layer "F.Cu") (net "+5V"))
 (segment (start 137.91 113.89) (end 163.1633 113.89) (width 0.2) (layer "F.Cu") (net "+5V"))
 (segment (start 164.5 114.5) (end 163.7733 114.5) (width 0.2) (layer "F.Cu") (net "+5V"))
 (segment (start 136.64 112.62) (end 137.91 113.89) (width 0.2) (layer "F.Cu") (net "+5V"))
 (segment (start 136.64 112.62) (end 136.64 110.08) (width 0.2) (layer "B.Cu") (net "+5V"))
 (segment (start 159.5 97.38) (end 165.5 103.38) (width 0.2) (layer "B.Cu") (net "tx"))
 (segment (start 165.5 103.38) (end 165.5 114.5) (width 0.2) (layer "B.Cu") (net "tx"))
 (segment (start 162.9141 114.1957) (end 163.9841 115.2657) (width 0.2) (layer "B.Cu") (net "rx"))
 (segment (start 159.5 99.92) (end 162.9141 103.3341) (width 0.2) (layer "B.Cu") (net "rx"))
 (segment (start 166.5 114.6264) (end 166.5 114.5) (width 0.2) (layer "B.Cu") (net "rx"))
 (segment (start 162.9141 103.3341) (end 162.9141 114.1957) (width 0.2) (layer "B.Cu") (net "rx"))
 (segment (start 165.8607 115.2657) (end 166.5 114.6264) (width 0.2) (layer "B.Cu") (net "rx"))
 (segment (start 163.9841 115.2657) (end 165.8607 115.2657) (width 0.2) (layer "B.Cu") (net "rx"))
 (segment (start 136.64 102.46) (end 148 91.1) (width 0.2) (layer "B.Cu") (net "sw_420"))
 (segment (start 148 91.1) (end 148 68) (width 0.2) (layer "B.Cu") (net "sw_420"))
 (segment (start 131.75 83.25) (end 125.25 83.25) (width 0.2) (layer "F.Cu") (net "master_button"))
 (segment (start 136.64 89.76) (end 131.75 84.87) (width 0.2) (layer "B.Cu") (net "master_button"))
 (segment (start 131.75 84.87) (end 131.75 83.25) (width 0.2) (layer "B.Cu") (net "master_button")))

